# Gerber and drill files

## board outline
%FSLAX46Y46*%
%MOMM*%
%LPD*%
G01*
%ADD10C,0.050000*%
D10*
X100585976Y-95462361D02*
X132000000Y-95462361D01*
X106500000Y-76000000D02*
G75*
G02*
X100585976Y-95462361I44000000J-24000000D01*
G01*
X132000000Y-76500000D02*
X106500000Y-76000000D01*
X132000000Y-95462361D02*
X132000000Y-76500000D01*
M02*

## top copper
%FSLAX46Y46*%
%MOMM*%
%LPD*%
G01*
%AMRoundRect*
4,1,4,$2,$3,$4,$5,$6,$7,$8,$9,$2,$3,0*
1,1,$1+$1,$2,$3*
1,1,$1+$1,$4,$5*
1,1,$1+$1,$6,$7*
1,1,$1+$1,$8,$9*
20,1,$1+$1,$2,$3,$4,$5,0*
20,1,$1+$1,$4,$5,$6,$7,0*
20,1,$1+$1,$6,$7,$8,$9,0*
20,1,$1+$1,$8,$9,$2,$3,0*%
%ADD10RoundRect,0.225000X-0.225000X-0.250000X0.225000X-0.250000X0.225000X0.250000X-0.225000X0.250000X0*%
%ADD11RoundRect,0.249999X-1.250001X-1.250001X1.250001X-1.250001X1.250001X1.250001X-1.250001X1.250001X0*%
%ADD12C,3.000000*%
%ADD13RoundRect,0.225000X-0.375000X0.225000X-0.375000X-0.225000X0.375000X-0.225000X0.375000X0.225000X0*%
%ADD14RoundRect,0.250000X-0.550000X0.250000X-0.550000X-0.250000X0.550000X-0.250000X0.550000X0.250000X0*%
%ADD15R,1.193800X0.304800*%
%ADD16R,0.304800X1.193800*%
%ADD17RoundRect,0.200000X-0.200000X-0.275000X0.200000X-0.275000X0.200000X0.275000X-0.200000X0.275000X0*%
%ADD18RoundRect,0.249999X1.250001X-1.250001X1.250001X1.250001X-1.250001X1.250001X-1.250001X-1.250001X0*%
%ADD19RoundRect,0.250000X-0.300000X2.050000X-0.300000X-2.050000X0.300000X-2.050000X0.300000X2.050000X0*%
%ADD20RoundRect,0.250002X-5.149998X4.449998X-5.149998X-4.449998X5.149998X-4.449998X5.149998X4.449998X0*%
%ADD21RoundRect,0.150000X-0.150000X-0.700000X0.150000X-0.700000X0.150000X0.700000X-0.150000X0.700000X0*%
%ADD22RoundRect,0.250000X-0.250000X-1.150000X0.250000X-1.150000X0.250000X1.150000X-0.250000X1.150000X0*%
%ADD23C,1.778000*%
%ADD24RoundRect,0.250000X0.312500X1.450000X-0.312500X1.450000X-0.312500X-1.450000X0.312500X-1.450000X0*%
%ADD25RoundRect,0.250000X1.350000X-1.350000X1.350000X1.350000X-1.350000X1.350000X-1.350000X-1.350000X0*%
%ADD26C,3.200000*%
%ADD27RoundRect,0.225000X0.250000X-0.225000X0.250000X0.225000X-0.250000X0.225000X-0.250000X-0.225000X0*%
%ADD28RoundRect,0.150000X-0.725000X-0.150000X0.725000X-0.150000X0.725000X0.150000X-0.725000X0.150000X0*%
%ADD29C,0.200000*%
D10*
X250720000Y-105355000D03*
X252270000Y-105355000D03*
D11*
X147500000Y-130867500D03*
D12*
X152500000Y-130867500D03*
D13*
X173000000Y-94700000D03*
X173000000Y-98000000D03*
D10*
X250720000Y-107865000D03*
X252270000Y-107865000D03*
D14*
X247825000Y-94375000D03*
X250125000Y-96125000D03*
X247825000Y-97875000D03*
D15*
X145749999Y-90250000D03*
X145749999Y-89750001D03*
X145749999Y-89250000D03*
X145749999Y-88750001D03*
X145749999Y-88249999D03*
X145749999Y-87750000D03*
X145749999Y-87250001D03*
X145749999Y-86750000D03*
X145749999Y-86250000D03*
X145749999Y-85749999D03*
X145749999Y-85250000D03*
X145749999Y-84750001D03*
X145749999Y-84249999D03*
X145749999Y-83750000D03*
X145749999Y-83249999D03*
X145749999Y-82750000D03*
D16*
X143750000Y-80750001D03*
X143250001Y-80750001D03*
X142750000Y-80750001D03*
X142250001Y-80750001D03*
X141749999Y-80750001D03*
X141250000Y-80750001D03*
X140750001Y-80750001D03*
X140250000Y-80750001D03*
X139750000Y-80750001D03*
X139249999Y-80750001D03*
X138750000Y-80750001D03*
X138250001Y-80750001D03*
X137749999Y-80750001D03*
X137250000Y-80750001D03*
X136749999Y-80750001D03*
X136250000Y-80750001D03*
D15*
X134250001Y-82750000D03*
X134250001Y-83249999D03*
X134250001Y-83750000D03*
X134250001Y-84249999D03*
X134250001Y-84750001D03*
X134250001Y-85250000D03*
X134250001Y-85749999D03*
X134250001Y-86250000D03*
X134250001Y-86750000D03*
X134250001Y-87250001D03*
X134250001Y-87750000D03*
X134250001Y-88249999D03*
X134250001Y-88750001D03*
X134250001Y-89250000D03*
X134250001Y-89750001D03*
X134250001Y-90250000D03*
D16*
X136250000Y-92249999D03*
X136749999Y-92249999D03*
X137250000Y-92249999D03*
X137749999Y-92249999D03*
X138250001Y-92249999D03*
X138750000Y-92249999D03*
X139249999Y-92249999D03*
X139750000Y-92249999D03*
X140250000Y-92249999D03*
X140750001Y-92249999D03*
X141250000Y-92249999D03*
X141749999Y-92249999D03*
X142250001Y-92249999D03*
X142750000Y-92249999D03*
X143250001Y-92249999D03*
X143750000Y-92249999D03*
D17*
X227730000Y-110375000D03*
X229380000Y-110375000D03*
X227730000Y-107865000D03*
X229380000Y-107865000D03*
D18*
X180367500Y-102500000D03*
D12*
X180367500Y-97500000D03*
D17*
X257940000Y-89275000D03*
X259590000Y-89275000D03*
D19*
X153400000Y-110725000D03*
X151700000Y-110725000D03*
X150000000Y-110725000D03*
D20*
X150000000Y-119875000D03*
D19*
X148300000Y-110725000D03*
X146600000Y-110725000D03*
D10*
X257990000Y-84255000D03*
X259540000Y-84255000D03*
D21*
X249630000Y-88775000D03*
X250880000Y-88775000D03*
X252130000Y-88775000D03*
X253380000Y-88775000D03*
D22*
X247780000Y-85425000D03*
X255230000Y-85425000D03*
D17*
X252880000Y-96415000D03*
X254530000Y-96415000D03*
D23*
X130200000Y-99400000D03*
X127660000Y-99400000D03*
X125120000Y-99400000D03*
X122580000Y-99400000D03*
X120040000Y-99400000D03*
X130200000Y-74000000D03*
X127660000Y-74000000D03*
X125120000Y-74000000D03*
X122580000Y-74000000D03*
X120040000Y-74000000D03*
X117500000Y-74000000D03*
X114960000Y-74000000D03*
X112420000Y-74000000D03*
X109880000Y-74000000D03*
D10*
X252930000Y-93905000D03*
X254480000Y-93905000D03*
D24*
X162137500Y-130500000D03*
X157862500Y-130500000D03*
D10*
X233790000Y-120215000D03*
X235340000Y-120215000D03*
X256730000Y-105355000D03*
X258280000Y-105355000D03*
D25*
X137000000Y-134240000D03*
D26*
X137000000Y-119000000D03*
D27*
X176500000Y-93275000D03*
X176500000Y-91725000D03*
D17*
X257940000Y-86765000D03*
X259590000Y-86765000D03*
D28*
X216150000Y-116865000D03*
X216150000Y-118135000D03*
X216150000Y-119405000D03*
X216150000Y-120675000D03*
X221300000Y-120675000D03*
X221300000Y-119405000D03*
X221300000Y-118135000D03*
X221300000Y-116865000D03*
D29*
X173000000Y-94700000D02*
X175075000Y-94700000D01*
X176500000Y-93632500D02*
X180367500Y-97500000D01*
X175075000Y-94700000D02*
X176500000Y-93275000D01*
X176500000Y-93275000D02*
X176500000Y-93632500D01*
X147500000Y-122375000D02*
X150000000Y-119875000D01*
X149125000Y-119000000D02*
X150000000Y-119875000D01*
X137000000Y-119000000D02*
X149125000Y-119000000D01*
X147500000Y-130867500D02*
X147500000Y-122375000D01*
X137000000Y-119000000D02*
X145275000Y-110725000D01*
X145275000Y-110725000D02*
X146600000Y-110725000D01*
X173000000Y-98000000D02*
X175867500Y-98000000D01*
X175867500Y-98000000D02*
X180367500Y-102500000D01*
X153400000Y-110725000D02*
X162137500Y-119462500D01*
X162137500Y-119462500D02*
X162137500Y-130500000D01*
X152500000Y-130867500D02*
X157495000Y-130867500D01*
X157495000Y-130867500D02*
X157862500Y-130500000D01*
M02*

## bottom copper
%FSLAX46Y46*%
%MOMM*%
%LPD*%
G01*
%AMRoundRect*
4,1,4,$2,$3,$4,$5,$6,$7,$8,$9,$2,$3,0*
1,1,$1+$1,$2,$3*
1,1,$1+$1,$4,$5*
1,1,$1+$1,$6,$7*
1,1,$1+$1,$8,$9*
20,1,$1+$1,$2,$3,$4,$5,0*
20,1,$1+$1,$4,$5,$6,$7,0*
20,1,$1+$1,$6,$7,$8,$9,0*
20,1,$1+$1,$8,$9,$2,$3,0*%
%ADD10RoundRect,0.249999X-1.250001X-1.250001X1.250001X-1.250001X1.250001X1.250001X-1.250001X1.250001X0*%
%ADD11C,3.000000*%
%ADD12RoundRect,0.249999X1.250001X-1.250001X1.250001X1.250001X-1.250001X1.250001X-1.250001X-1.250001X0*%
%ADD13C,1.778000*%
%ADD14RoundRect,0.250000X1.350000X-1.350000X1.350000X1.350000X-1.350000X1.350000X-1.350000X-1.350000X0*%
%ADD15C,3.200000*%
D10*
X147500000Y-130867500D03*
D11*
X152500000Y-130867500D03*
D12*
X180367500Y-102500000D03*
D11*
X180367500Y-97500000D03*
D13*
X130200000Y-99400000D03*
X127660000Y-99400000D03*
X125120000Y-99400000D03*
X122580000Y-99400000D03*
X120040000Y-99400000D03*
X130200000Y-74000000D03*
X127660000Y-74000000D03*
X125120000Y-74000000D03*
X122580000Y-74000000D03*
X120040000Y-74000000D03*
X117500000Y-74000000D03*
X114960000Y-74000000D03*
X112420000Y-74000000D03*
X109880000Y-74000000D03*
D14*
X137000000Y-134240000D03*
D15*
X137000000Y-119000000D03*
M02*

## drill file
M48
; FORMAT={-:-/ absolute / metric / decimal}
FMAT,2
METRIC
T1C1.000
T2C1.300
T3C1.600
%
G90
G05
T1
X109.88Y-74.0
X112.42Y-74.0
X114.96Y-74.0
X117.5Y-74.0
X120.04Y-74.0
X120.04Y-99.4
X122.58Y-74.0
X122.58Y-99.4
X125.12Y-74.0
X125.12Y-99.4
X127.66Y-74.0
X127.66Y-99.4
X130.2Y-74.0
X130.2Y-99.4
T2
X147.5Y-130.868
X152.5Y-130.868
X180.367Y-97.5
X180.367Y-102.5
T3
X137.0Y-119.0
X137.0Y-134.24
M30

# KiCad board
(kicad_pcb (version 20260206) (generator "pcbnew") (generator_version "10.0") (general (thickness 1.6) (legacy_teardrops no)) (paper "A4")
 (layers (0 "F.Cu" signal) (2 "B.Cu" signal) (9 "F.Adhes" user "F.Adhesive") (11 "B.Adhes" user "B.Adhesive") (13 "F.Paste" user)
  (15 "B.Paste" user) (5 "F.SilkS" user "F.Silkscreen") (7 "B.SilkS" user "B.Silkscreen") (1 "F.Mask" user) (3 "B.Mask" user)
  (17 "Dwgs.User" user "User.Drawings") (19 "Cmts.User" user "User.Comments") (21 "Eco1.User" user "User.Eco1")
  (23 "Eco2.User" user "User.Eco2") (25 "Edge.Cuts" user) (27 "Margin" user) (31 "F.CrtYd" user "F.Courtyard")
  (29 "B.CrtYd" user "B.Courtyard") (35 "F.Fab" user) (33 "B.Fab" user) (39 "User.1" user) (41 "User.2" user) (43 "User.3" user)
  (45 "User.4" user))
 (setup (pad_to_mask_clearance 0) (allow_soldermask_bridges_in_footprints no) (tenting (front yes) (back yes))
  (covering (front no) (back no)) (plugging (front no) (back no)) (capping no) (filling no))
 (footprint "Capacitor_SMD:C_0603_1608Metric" (layer "F.Cu") (at 251.495 105.355)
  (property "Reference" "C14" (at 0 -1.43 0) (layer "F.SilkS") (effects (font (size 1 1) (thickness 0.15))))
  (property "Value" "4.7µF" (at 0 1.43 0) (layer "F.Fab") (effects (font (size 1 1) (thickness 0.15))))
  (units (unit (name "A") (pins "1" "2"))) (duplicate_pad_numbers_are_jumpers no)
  (pad "1" smd roundrect (at -0.775 0) (size 0.9 0.95) (layers "F.Cu" "F.Mask" "F.Paste") (roundrect_rratio 0.25) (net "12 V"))
  (pad "2" smd roundrect (at 0.775 0) (size 0.9 0.95) (layers "F.Cu" "F.Mask" "F.Paste") (roundrect_rratio 0.25) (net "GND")))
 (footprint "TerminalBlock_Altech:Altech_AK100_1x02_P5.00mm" (layer "F.Cu") (at 147.5 130.8675)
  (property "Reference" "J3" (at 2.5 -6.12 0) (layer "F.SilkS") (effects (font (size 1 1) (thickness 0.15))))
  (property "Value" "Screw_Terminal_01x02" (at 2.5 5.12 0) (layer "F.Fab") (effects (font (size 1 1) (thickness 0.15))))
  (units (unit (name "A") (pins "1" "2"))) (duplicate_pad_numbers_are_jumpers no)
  (pad "1" thru_hole roundrect (at 0 0) (size 3 3) (drill 1.3) (layers "*.Cu" "*.Mask") (remove_unused_layers no)
   (roundrect_rratio 0.083333) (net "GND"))
  (pad "2" thru_hole circle (at 5 0) (size 3 3) (drill 1.3) (layers "*.Cu" "*.Mask") (remove_unused_layers no) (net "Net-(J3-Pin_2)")))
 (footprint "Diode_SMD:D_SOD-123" (layer "F.Cu") (at 173 96.35 -90)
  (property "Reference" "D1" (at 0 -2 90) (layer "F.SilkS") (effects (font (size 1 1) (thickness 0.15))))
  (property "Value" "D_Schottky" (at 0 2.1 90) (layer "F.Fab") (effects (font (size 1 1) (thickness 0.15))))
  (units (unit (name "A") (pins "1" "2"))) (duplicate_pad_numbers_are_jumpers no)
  (pad "1" smd roundrect (at -1.65 0 270) (size 0.9 1.2) (layers "F.Cu" "F.Mask" "F.Paste") (roundrect_rratio 0.25) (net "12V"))
  (pad "2" smd roundrect (at 1.65 0 270) (size 0.9 1.2) (layers "F.Cu" "F.Mask" "F.Paste") (roundrect_rratio 0.25) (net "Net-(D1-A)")))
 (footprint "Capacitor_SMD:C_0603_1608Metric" (layer "F.Cu") (at 251.495 107.865)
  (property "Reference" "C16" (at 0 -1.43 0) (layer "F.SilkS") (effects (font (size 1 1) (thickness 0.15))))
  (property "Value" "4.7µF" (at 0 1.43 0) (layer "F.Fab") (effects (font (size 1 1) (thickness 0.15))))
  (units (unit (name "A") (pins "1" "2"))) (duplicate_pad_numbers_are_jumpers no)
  (pad "1" smd roundrect (at -0.775 0) (size 0.9 0.95) (layers "F.Cu" "F.Mask" "F.Paste") (roundrect_rratio 0.25) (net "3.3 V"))
  (pad "2" smd roundrect (at 0.775 0) (size 0.9 0.95) (layers "F.Cu" "F.Mask" "F.Paste") (roundrect_rratio 0.25) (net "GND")))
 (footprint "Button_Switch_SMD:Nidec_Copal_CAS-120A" (layer "F.Cu") (at 248.975 96.125)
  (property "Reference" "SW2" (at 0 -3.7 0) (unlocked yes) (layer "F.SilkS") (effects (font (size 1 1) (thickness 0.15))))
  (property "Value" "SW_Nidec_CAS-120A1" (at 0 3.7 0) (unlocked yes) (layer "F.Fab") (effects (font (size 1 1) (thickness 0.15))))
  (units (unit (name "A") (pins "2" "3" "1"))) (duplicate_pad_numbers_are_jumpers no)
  (pad "1" smd roundrect (at -1.15 -1.75 270) (size 1 1.6) (layers "F.Cu" "F.Mask" "F.Paste") (roundrect_rratio 0.25) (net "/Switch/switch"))
  (pad "2" smd roundrect (at 1.15 0 270) (size 1 1.6) (layers "F.Cu" "F.Mask" "F.Paste") (roundrect_rratio 0.25) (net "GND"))
  (pad "3" smd roundrect (at -1.15 1.75 270) (size 1 1.6) (layers "F.Cu" "F.Mask" "F.Paste") (roundrect_rratio 0.25)
   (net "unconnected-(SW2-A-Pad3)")))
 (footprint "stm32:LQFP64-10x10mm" (layer "F.Cu") (at 140 86.5 180)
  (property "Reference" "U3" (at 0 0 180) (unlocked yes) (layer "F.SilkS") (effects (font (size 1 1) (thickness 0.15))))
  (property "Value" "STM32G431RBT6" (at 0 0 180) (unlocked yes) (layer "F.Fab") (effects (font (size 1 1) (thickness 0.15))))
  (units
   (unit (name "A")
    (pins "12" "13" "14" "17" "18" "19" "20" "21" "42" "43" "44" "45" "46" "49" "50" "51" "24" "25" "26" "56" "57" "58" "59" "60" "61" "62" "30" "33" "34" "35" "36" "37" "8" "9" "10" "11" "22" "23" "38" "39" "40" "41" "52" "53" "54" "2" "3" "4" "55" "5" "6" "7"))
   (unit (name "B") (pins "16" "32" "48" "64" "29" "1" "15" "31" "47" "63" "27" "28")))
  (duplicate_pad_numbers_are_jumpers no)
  (pad "1" smd rect (at -5.749999 -3.75 180) (size 1.1938 0.3048) (layers "F.Cu" "F.Mask" "F.Paste") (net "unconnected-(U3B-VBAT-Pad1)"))
  (pad "2" smd rect (at -5.749999 -3.250001 180) (size 1.1938 0.3048) (layers "F.Cu" "F.Mask" "F.Paste") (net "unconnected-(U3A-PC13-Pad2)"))
  (pad "3" smd rect (at -5.749999 -2.75 180) (size 1.1938 0.3048) (layers "F.Cu" "F.Mask" "F.Paste")
   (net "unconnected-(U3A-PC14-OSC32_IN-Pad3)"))
  (pad "4" smd rect (at -5.749999 -2.250001 180) (size 1.1938 0.3048) (layers "F.Cu" "F.Mask" "F.Paste")
   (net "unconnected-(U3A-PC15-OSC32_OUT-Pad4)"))
  (pad "5" smd rect (at -5.749999 -1.749999 180) (size 1.1938 0.3048) (layers "F.Cu" "F.Mask" "F.Paste")
   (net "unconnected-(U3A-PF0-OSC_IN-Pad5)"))
  (pad "6" smd rect (at -5.749999 -1.25 180) (size 1.1938 0.3048) (layers "F.Cu" "F.Mask" "F.Paste")
   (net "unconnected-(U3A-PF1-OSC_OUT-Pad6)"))
  (pad "7" smd rect (at -5.749999 -0.750001 180) (size 1.1938 0.3048) (layers "F.Cu" "F.Mask" "F.Paste")
   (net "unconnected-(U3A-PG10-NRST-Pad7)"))
  (pad "8" smd rect (at -5.749999 -0.25 180) (size 1.1938 0.3048) (layers "F.Cu" "F.Mask" "F.Paste") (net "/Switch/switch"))
  (pad "9" smd rect (at -5.749999 0.25 180) (size 1.1938 0.3048) (layers "F.Cu" "F.Mask" "F.Paste") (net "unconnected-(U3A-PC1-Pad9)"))
  (pad "10" smd rect (at -5.749999 0.750001 180) (size 1.1938 0.3048) (layers "F.Cu" "F.Mask" "F.Paste") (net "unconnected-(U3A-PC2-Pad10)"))
  (pad "11" smd rect (at -5.749999 1.25 180) (size 1.1938 0.3048) (layers "F.Cu" "F.Mask" "F.Paste") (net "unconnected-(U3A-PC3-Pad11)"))
  (pad "12" smd rect (at -5.749999 1.749999 180) (size 1.1938 0.3048) (layers "F.Cu" "F.Mask" "F.Paste") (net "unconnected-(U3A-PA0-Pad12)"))
  (pad "13" smd rect (at -5.749999 2.250001 180) (size 1.1938 0.3048) (layers "F.Cu" "F.Mask" "F.Paste") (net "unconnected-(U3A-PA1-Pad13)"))
  (pad "14" smd rect (at -5.749999 2.75 180) (size 1.1938 0.3048) (layers "F.Cu" "F.Mask" "F.Paste") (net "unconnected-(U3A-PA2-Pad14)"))
  (pad "15" smd rect (at -5.749999 3.250001 180) (size 1.1938 0.3048) (layers "F.Cu" "F.Mask" "F.Paste") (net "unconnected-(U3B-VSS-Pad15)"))
  (pad "16" smd rect (at -5.749999 3.75 180) (size 1.1938 0.3048) (layers "F.Cu" "F.Mask" "F.Paste") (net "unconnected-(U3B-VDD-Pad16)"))
  (pad "17" smd rect (at -3.75 5.749999 270) (size 1.1938 0.3048) (layers "F.Cu" "F.Mask" "F.Paste") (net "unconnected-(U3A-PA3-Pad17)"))
  (pad "18" smd rect (at -3.250001 5.749999 270) (size 1.1938 0.3048) (layers "F.Cu" "F.Mask" "F.Paste") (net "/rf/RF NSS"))
  (pad "19" smd rect (at -2.75 5.749999 270) (size 1.1938 0.3048) (layers "F.Cu" "F.Mask" "F.Paste") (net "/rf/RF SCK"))
  (pad "20" smd rect (at -2.250001 5.749999 270) (size 1.1938 0.3048) (layers "F.Cu" "F.Mask" "F.Paste") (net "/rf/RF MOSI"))
  (pad "21" smd rect (at -1.749999 5.749999 270) (size 1.1938 0.3048) (layers "F.Cu" "F.Mask" "F.Paste") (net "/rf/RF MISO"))
  (pad "22" smd rect (at -1.25 5.749999 270) (size 1.1938 0.3048) (layers "F.Cu" "F.Mask" "F.Paste") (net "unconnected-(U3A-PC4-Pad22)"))
  (pad "23" smd rect (at -0.750001 5.749999 270) (size 1.1938 0.3048) (layers "F.Cu" "F.Mask" "F.Paste") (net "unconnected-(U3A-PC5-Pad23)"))
  (pad "24" smd rect (at -0.25 5.749999 270) (size 1.1938 0.3048) (layers "F.Cu" "F.Mask" "F.Paste") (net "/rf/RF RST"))
  (pad "25" smd rect (at 0.25 5.749999 270) (size 1.1938 0.3048) (layers "F.Cu" "F.Mask" "F.Paste") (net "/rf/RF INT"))
  (pad "26" smd rect (at 0.750001 5.749999 270) (size 1.1938 0.3048) (layers "F.Cu" "F.Mask" "F.Paste") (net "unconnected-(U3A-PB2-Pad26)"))
  (pad "27" smd rect (at 1.25 5.749999 270) (size 1.1938 0.3048) (layers "F.Cu" "F.Mask" "F.Paste") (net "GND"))
  (pad "28" smd rect (at 1.749999 5.749999 270) (size 1.1938 0.3048) (layers "F.Cu" "F.Mask" "F.Paste") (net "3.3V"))
  (pad "29" smd rect (at 2.250001 5.749999 270) (size 1.1938 0.3048) (layers "F.Cu" "F.Mask" "F.Paste") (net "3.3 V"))
  (pad "30" smd rect (at 2.75 5.749999 270) (size 1.1938 0.3048) (layers "F.Cu" "F.Mask" "F.Paste") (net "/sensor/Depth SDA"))
  (pad "31" smd rect (at 3.250001 5.749999 270) (size 1.1938 0.3048) (layers "F.Cu" "F.Mask" "F.Paste") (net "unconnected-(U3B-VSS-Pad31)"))
  (pad "32" smd rect (at 3.75 5.749999 270) (size 1.1938 0.3048) (layers "F.Cu" "F.Mask" "F.Paste") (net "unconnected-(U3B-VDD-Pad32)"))
  (pad "33" smd rect (at 5.749999 3.75 180) (size 1.1938 0.3048) (layers "F.Cu" "F.Mask" "F.Paste") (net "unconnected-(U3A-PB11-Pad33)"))
  (pad "34" smd rect (at 5.749999 3.250001 180) (size 1.1938 0.3048) (layers "F.Cu" "F.Mask" "F.Paste") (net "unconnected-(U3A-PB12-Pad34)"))
  (pad "35" smd rect (at 5.749999 2.75 180) (size 1.1938 0.3048) (layers "F.Cu" "F.Mask" "F.Paste") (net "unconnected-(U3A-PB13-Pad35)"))
  (pad "36" smd rect (at 5.749999 2.250001 180) (size 1.1938 0.3048) (layers "F.Cu" "F.Mask" "F.Paste") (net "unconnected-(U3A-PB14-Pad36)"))
  (pad "37" smd rect (at 5.749999 1.749999 180) (size 1.1938 0.3048) (layers "F.Cu" "F.Mask" "F.Paste") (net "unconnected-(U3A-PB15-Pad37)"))
  (pad "38" smd rect (at 5.749999 1.25 180) (size 1.1938 0.3048) (layers "F.Cu" "F.Mask" "F.Paste") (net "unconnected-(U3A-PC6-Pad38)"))
  (pad "39" smd rect (at 5.749999 0.750001 180) (size 1.1938 0.3048) (layers "F.Cu" "F.Mask" "F.Paste") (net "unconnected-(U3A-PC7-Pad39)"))
  (pad "40" smd rect (at 5.749999 0.25 180) (size 1.1938 0.3048) (layers "F.Cu" "F.Mask" "F.Paste") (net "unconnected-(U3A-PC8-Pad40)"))
  (pad "41" smd rect (at 5.749999 -0.25 180) (size 1.1938 0.3048) (layers "F.Cu" "F.Mask" "F.Paste") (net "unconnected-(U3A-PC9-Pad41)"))
  (pad "42" smd rect (at 5.749999 -0.750001 180) (size 1.1938 0.3048) (layers "F.Cu" "F.Mask" "F.Paste") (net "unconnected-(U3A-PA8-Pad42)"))
  (pad "43" smd rect (at 5.749999 -1.25 180) (size 1.1938 0.3048) (layers "F.Cu" "F.Mask" "F.Paste") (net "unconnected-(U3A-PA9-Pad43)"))
  (pad "44" smd rect (at 5.749999 -1.749999 180) (size 1.1938 0.3048) (layers "F.Cu" "F.Mask" "F.Paste") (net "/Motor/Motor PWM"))
  (pad "45" smd rect (at 5.749999 -2.250001 180) (size 1.1938 0.3048) (layers "F.Cu" "F.Mask" "F.Paste")
   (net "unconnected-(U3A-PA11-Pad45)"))
  (pad "46" smd rect (at 5.749999 -2.75 180) (size 1.1938 0.3048) (layers "F.Cu" "F.Mask" "F.Paste") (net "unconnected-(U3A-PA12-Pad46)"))
  (pad "47" smd rect (at 5.749999 -3.250001 180) (size 1.1938 0.3048) (layers "F.Cu" "F.Mask" "F.Paste") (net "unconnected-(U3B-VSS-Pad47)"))
  (pad "48" smd rect (at 5.749999 -3.75 180) (size 1.1938 0.3048) (layers "F.Cu" "F.Mask" "F.Paste") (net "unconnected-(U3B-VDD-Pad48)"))
  (pad "49" smd rect (at 3.75 -5.749999 270) (size 1.1938 0.3048) (layers "F.Cu" "F.Mask" "F.Paste") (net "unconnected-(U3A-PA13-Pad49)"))
  (pad "50" smd rect (at 3.250001 -5.749999 270) (size 1.1938 0.3048) (layers "F.Cu" "F.Mask" "F.Paste")
   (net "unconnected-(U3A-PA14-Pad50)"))
  (pad "51" smd rect (at 2.75 -5.749999 270) (size 1.1938 0.3048) (layers "F.Cu" "F.Mask" "F.Paste") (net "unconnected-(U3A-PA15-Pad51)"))
  (pad "52" smd rect (at 2.250001 -5.749999 270) (size 1.1938 0.3048) (layers "F.Cu" "F.Mask" "F.Paste")
   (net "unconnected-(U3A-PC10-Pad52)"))
  (pad "53" smd rect (at 1.749999 -5.749999 270) (size 1.1938 0.3048) (layers "F.Cu" "F.Mask" "F.Paste")
   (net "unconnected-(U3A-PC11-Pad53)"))
  (pad "54" smd rect (at 1.25 -5.749999 270) (size 1.1938 0.3048) (layers "F.Cu" "F.Mask" "F.Paste") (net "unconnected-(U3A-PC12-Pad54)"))
  (pad "55" smd rect (at 0.750001 -5.749999 270) (size 1.1938 0.3048) (layers "F.Cu" "F.Mask" "F.Paste") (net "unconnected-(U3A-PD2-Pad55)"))
  (pad "56" smd rect (at 0.25 -5.749999 270) (size 1.1938 0.3048) (layers "F.Cu" "F.Mask" "F.Paste") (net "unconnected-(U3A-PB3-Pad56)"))
  (pad "57" smd rect (at -0.25 -5.749999 270) (size 1.1938 0.3048) (layers "F.Cu" "F.Mask" "F.Paste") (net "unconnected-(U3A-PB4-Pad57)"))
  (pad "58" smd rect (at -0.750001 -5.749999 270) (size 1.1938 0.3048) (layers "F.Cu" "F.Mask" "F.Paste")
   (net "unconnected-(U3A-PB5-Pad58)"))
  (pad "59" smd rect (at -1.25 -5.749999 270) (size 1.1938 0.3048) (layers "F.Cu" "F.Mask" "F.Paste") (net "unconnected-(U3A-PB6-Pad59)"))
  (pad "60" smd rect (at -1.749999 -5.749999 270) (size 1.1938 0.3048) (layers "F.Cu" "F.Mask" "F.Paste")
   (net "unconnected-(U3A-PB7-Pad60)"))
  (pad "61" smd rect (at -2.250001 -5.749999 270) (size 1.1938 0.3048) (layers "F.Cu" "F.Mask" "F.Paste")
   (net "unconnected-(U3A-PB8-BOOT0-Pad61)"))
  (pad "62" smd rect (at -2.75 -5.749999 270) (size 1.1938 0.3048) (layers "F.Cu" "F.Mask" "F.Paste") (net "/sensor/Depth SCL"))
  (pad "63" smd rect (at -3.250001 -5.749999 270) (size 1.1938 0.3048) (layers "F.Cu" "F.Mask" "F.Paste") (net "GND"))
  (pad "64" smd rect (at -3.75 -5.749999 270) (size 1.1938 0.3048) (layers "F.Cu" "F.Mask" "F.Paste") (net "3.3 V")))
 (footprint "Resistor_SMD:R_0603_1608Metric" (layer "F.Cu") (at 228.555 110.375)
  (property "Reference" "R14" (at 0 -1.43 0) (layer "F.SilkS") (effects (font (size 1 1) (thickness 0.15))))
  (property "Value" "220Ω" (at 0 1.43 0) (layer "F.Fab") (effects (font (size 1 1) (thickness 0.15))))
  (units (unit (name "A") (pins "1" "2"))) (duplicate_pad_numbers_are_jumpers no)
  (pad "1" smd roundrect (at -0.825 0) (size 0.8 0.95) (layers "F.Cu" "F.Mask" "F.Paste") (roundrect_rratio 0.25) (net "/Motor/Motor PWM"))
  (pad "2" smd roundrect (at 0.825 0) (size 0.8 0.95) (layers "F.Cu" "F.Mask" "F.Paste") (roundrect_rratio 0.25) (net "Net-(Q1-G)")))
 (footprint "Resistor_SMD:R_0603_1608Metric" (layer "F.Cu") (at 228.555 107.865)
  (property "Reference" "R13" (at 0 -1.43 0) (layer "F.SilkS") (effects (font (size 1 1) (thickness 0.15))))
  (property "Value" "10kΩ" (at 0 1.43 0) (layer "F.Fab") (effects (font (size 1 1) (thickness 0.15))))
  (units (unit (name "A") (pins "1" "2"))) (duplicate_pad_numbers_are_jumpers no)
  (pad "1" smd roundrect (at -0.825 0) (size 0.8 0.95) (layers "F.Cu" "F.Mask" "F.Paste") (roundrect_rratio 0.25) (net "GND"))
  (pad "2" smd roundrect (at 0.825 0) (size 0.8 0.95) (layers "F.Cu" "F.Mask" "F.Paste") (roundrect_rratio 0.25) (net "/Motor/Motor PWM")))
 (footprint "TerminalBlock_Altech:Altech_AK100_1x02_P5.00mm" (layer "F.Cu") (at 180.3675 102.5 90)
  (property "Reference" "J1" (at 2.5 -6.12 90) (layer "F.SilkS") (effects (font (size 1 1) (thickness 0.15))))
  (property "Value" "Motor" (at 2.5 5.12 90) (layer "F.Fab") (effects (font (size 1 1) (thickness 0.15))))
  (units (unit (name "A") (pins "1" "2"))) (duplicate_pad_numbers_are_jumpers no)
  (pad "1" thru_hole roundrect (at 0 0 90) (size 3 3) (drill 1.3) (layers "*.Cu" "*.Mask") (remove_unused_layers no)
   (roundrect_rratio 0.083333) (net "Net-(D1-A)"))
  (pad "2" thru_hole circle (at 5 0 90) (size 3 3) (drill 1.3) (layers "*.Cu" "*.Mask") (remove_unused_layers no) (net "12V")))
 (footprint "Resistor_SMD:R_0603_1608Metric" (layer "F.Cu") (at 258.765 89.275)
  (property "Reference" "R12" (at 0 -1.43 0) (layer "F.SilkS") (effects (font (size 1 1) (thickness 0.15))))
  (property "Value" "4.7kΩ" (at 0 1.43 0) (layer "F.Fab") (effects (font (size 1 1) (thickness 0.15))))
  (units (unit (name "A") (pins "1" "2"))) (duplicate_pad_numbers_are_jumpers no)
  (pad "1" smd roundrect (at -0.825 0) (size 0.8 0.95) (layers "F.Cu" "F.Mask" "F.Paste") (roundrect_rratio 0.25) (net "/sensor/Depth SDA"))
  (pad "2" smd roundrect (at 0.825 0) (size 0.8 0.95) (layers "F.Cu" "F.Mask" "F.Paste") (roundrect_rratio 0.25) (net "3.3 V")))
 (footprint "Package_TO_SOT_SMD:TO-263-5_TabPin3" (layer "F.Cu") (at 150 118.375 -90)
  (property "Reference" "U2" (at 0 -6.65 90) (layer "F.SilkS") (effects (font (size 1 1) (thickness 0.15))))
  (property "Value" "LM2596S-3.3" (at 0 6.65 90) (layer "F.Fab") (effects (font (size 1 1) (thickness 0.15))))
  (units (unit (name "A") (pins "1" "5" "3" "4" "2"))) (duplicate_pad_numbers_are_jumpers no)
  (pad "" smd roundrect (at -0.925 -2.775 270) (size 4.55 5.25) (layers "F.Paste") (roundrect_rratio 0.054945))
  (pad "" smd roundrect (at -0.925 2.775 270) (size 4.55 5.25) (layers "F.Paste") (roundrect_rratio 0.054945))
  (pad "" smd roundrect (at 3.925 -2.775 270) (size 4.55 5.25) (layers "F.Paste") (roundrect_rratio 0.054945))
  (pad "" smd roundrect (at 3.925 2.775 270) (size 4.55 5.25) (layers "F.Paste") (roundrect_rratio 0.054945))
  (pad "1" smd roundrect (at -7.65 -3.4 270) (size 4.6 1.1) (layers "F.Cu" "F.Mask" "F.Paste") (roundrect_rratio 0.227273) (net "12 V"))
  (pad "2" smd roundrect (at -7.65 -1.7 270) (size 4.6 1.1) (layers "F.Cu" "F.Mask" "F.Paste") (roundrect_rratio 0.227273)
   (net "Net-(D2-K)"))
  (pad "3" smd roundrect (at -7.65 0 270) (size 4.6 1.1) (layers "F.Cu" "F.Mask" "F.Paste") (roundrect_rratio 0.227273) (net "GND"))
  (pad "3" smd roundrect (at 1.5 0 270) (size 9.4 10.8) (layers "F.Cu" "F.Mask") (roundrect_rratio 0.026596) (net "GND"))
  (pad "4" smd roundrect (at -7.65 1.7 270) (size 4.6 1.1) (layers "F.Cu" "F.Mask" "F.Paste") (roundrect_rratio 0.227273) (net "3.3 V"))
  (pad "5" smd roundrect (at -7.65 3.4 270) (size 4.6 1.1) (layers "F.Cu" "F.Mask" "F.Paste") (roundrect_rratio 0.227273) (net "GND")))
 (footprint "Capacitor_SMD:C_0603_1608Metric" (layer "F.Cu") (at 258.765 84.255)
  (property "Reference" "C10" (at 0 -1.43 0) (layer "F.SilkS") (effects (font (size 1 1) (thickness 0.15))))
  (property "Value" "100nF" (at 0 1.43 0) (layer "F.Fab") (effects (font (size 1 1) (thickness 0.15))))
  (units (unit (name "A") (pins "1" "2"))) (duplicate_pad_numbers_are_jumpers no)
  (pad "1" smd roundrect (at -0.775 0) (size 0.9 0.95) (layers "F.Cu" "F.Mask" "F.Paste") (roundrect_rratio 0.25) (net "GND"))
  (pad "2" smd roundrect (at 0.775 0) (size 0.9 0.95) (layers "F.Cu" "F.Mask" "F.Paste") (roundrect_rratio 0.25) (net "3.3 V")))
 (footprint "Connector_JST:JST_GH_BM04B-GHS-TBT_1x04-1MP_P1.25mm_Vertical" (layer "F.Cu") (at 251.505 86.825)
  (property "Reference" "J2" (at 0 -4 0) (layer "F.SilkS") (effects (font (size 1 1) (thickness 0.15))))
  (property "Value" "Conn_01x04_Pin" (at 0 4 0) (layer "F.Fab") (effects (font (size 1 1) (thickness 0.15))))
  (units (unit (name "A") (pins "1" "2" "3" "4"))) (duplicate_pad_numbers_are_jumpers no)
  (pad "1" smd roundrect (at -1.875 1.95) (size 0.6 1.7) (layers "F.Cu" "F.Mask" "F.Paste") (roundrect_rratio 0.25) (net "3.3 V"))
  (pad "2" smd roundrect (at -0.625 1.95) (size 0.6 1.7) (layers "F.Cu" "F.Mask" "F.Paste") (roundrect_rratio 0.25)
   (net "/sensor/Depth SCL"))
  (pad "3" smd roundrect (at 0.625 1.95) (size 0.6 1.7) (layers "F.Cu" "F.Mask" "F.Paste") (roundrect_rratio 0.25) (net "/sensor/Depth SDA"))
  (pad "4" smd roundrect (at 1.875 1.95) (size 0.6 1.7) (layers "F.Cu" "F.Mask" "F.Paste") (roundrect_rratio 0.25) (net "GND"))
  (pad "MP" smd roundrect (at -3.725 -1.4) (size 1 2.8) (layers "F.Cu" "F.Mask" "F.Paste") (roundrect_rratio 0.25))
  (pad "MP" smd roundrect (at 3.725 -1.4) (size 1 2.8) (layers "F.Cu" "F.Mask" "F.Paste") (roundrect_rratio 0.25)))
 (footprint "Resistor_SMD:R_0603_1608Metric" (layer "F.Cu") (at 253.705 96.415)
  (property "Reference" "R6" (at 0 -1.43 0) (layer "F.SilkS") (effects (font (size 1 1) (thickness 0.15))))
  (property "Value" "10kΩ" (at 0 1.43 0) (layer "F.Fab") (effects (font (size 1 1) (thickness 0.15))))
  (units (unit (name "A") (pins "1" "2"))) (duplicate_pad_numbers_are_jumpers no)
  (pad "1" smd roundrect (at -0.825 0) (size 0.8 0.95) (layers "F.Cu" "F.Mask" "F.Paste") (roundrect_rratio 0.25) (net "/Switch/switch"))
  (pad "2" smd roundrect (at 0.825 0) (size 0.8 0.95) (layers "F.Cu" "F.Mask" "F.Paste") (roundrect_rratio 0.25) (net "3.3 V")))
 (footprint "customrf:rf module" (layer "F.Cu") (at 130.2 99.4 180)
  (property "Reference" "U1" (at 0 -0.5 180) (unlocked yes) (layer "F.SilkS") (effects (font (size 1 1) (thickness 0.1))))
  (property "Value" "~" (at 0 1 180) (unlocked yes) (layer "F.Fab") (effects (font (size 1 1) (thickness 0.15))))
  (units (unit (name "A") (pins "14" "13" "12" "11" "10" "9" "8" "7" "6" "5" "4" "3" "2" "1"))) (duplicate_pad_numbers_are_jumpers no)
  (pad "1" thru_hole circle (at 0 0 270) (size 1.778 1.778) (drill 1) (layers "*.Cu" "*.Mask") (remove_unused_layers no)
   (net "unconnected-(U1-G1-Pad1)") (solder_mask_margin 0.0508) (thermal_bridge_angle 0))
  (pad "2" thru_hole circle (at 2.54 0 270) (size 1.778 1.778) (drill 1) (layers "*.Cu" "*.Mask") (remove_unused_layers no)
   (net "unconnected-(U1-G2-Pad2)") (solder_mask_margin 0.0508) (thermal_bridge_angle 0))
  (pad "3" thru_hole circle (at 5.08 0 270) (size 1.778 1.778) (drill 1) (layers "*.Cu" "*.Mask") (remove_unused_layers no)
   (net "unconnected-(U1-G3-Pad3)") (solder_mask_margin 0.0508) (thermal_bridge_angle 0))
  (pad "4" thru_hole circle (at 7.62 0 270) (size 1.778 1.778) (drill 1) (layers "*.Cu" "*.Mask") (remove_unused_layers no)
   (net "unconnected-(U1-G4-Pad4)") (solder_mask_margin 0.0508) (thermal_bridge_angle 0))
  (pad "5" thru_hole circle (at 10.16 0 270) (size 1.778 1.778) (drill 1) (layers "*.Cu" "*.Mask") (remove_unused_layers no)
   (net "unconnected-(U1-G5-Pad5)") (solder_mask_margin 0.0508) (thermal_bridge_angle 0))
  (pad "6" thru_hole circle (at 0 25.4 270) (size 1.778 1.778) (drill 1) (layers "*.Cu" "*.Mask") (remove_unused_layers no) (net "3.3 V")
   (solder_mask_margin 0.0508) (thermal_bridge_angle 0))
  (pad "7" thru_hole circle (at 2.54 25.4 270) (size 1.778 1.778) (drill 1) (layers "*.Cu" "*.Mask") (remove_unused_layers no) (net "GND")
   (solder_mask_margin 0.0508) (thermal_bridge_angle 0))
  (pad "8" thru_hole circle (at 5.08 25.4 270) (size 1.778 1.778) (drill 1) (layers "*.Cu" "*.Mask") (remove_unused_layers no)
   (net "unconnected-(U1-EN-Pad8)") (solder_mask_margin 0.0508) (thermal_bridge_angle 0))
  (pad "9" thru_hole circle (at 7.62 25.4 270) (size 1.778 1.778) (drill 1) (layers "*.Cu" "*.Mask") (remove_unused_layers no)
   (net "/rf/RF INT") (solder_mask_margin 0.0508) (thermal_bridge_angle 0))
  (pad "10" thru_hole circle (at 10.16 25.4 270) (size 1.778 1.778) (drill 1) (layers "*.Cu" "*.Mask") (remove_unused_layers no)
   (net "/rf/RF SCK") (solder_mask_margin 0.0508) (thermal_bridge_angle 0))
  (pad "11" thru_hole circle (at 12.7 25.4 270) (size 1.778 1.778) (drill 1) (layers "*.Cu" "*.Mask") (remove_unused_layers no)
   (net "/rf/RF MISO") (solder_mask_margin 0.0508) (thermal_bridge_angle 0))
  (pad "12" thru_hole circle (at 15.24 25.4 270) (size 1.778 1.778) (drill 1) (layers "*.Cu" "*.Mask") (remove_unused_layers no)
   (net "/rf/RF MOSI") (solder_mask_margin 0.0508) (thermal_bridge_angle 0))
  (pad "13" thru_hole circle (at 17.78 25.4 270) (size 1.778 1.778) (drill 1) (layers "*.Cu" "*.Mask") (remove_unused_layers no)
   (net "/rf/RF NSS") (solder_mask_margin 0.0508) (thermal_bridge_angle 0))
  (pad "14" thru_hole circle (at 20.32 25.4 270) (size 1.778 1.778) (drill 1) (layers "*.Cu" "*.Mask") (remove_unused_layers no)
   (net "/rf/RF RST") (solder_mask_margin 0.0508) (thermal_bridge_angle 0)))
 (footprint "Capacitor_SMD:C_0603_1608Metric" (layer "F.Cu") (at 253.705 93.905)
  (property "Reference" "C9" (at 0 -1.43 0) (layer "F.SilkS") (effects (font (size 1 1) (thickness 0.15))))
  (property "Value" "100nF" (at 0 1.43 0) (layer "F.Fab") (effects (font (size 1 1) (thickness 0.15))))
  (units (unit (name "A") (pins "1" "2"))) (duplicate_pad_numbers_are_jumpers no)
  (pad "1" smd roundrect (at -0.775 0) (size 0.9 0.95) (layers "F.Cu" "F.Mask" "F.Paste") (roundrect_rratio 0.25) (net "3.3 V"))
  (pad "2" smd roundrect (at 0.775 0) (size 0.9 0.95) (layers "F.Cu" "F.Mask" "F.Paste") (roundrect_rratio 0.25) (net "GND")))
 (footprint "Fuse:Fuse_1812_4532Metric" (layer "F.Cu") (at 160 130.5 180)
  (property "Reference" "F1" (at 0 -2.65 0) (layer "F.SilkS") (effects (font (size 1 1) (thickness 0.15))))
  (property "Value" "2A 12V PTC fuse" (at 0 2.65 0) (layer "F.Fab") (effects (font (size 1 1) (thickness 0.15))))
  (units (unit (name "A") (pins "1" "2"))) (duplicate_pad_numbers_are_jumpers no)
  (pad "1" smd roundrect (at -2.1375 0 180) (size 1.125 3.4) (layers "F.Cu" "F.Mask" "F.Paste") (roundrect_rratio 0.222222) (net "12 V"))
  (pad "2" smd roundrect (at 2.1375 0 180) (size 1.125 3.4) (layers "F.Cu" "F.Mask" "F.Paste") (roundrect_rratio 0.222222)
   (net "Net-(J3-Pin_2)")))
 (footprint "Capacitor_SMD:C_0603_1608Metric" (layer "F.Cu") (at 234.565 120.215)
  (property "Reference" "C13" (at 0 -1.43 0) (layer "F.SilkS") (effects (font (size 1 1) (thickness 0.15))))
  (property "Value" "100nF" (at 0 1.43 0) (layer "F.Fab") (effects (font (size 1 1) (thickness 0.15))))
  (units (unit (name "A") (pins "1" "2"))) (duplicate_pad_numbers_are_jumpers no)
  (pad "1" smd roundrect (at -0.775 0) (size 0.9 0.95) (layers "F.Cu" "F.Mask" "F.Paste") (roundrect_rratio 0.25) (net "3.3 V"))
  (pad "2" smd roundrect (at 0.775 0) (size 0.9 0.95) (layers "F.Cu" "F.Mask" "F.Paste") (roundrect_rratio 0.25) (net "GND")))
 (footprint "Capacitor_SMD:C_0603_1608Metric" (layer "F.Cu") (at 257.505 105.355)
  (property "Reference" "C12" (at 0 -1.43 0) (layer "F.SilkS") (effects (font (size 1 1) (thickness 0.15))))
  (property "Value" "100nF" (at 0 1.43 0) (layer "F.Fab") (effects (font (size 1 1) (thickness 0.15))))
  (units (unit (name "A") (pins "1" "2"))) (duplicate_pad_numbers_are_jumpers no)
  (pad "1" smd roundrect (at -0.775 0) (size 0.9 0.95) (layers "F.Cu" "F.Mask" "F.Paste") (roundrect_rratio 0.25) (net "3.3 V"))
  (pad "2" smd roundrect (at 0.775 0) (size 0.9 0.95) (layers "F.Cu" "F.Mask" "F.Paste") (roundrect_rratio 0.25) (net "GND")))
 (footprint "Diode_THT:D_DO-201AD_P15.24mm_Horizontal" (layer "F.Cu") (at 137 134.24 90)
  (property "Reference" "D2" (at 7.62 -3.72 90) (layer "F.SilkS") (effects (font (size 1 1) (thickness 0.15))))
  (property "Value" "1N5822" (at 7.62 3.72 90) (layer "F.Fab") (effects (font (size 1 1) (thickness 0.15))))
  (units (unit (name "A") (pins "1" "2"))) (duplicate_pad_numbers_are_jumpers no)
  (pad "1" thru_hole roundrect (at 0 0 90) (size 3.2 3.2) (drill 1.6) (layers "*.Cu" "*.Mask") (remove_unused_layers no)
   (roundrect_rratio 0.078125) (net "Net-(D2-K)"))
  (pad "2" thru_hole circle (at 15.24 0 90) (size 3.2 3.2) (drill 1.6) (layers "*.Cu" "*.Mask") (remove_unused_layers no) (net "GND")))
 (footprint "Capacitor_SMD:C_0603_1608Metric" (layer "F.Cu") (at 176.5 92.5 90)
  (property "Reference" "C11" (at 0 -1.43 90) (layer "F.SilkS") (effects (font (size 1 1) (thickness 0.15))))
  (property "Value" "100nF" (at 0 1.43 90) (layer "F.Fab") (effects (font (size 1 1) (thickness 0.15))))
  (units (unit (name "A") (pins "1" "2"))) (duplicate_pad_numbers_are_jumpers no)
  (pad "1" smd roundrect (at -0.775 0 90) (size 0.9 0.95) (layers "F.Cu" "F.Mask" "F.Paste") (roundrect_rratio 0.25) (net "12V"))
  (pad "2" smd roundrect (at 0.775 0 90) (size 0.9 0.95) (layers "F.Cu" "F.Mask" "F.Paste") (roundrect_rratio 0.25) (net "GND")))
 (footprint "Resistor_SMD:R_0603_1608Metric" (layer "F.Cu") (at 258.765 86.765)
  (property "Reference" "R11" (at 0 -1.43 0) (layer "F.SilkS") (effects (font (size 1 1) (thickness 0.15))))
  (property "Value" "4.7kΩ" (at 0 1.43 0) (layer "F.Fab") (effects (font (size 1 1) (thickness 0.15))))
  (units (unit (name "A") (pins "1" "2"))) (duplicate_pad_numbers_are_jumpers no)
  (pad "1" smd roundrect (at -0.825 0) (size 0.8 0.95) (layers "F.Cu" "F.Mask" "F.Paste") (roundrect_rratio 0.25) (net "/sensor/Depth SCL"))
  (pad "2" smd roundrect (at 0.825 0) (size 0.8 0.95) (layers "F.Cu" "F.Mask" "F.Paste") (roundrect_rratio 0.25) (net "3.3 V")))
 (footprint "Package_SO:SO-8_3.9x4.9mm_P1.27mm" (layer "F.Cu") (at 218.725 118.77)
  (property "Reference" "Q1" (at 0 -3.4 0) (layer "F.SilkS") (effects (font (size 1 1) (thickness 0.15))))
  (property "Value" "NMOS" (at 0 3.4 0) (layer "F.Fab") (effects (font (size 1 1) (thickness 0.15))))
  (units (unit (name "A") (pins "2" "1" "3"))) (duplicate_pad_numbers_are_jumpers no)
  (pad "1" smd roundrect (at -2.575 -1.905) (size 1.75 0.6) (layers "F.Cu" "F.Mask" "F.Paste") (roundrect_rratio 0.25) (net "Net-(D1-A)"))
  (pad "2" smd roundrect (at -2.575 -0.635) (size 1.75 0.6) (layers "F.Cu" "F.Mask" "F.Paste") (roundrect_rratio 0.25) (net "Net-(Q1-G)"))
  (pad "3" smd roundrect (at -2.575 0.635) (size 1.75 0.6) (layers "F.Cu" "F.Mask" "F.Paste") (roundrect_rratio 0.25) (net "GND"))
  (pad "4" smd roundrect (at -2.575 1.905) (size 1.75 0.6) (layers "F.Cu" "F.Mask" "F.Paste") (roundrect_rratio 0.25))
  (pad "5" smd roundrect (at 2.575 1.905) (size 1.75 0.6) (layers "F.Cu" "F.Mask" "F.Paste") (roundrect_rratio 0.25))
  (pad "6" smd roundrect (at 2.575 0.635) (size 1.75 0.6) (layers "F.Cu" "F.Mask" "F.Paste") (roundrect_rratio 0.25))
  (pad "7" smd roundrect (at 2.575 -0.635) (size 1.75 0.6) (layers "F.Cu" "F.Mask" "F.Paste") (roundrect_rratio 0.25))
  (pad "8" smd roundrect (at 2.575 -1.905) (size 1.75 0.6) (layers "F.Cu" "F.Mask" "F.Paste") (roundrect_rratio 0.25)))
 (gr_line (start 100.585976 95.462361) (end 132 95.462361) (stroke (width 0.05) (type default)) (layer "Edge.Cuts"))
 (gr_arc (start 106.5 76) (mid 198.454738 114.571998) (end 100.585976 95.462361) (stroke (width 0.05) (type default)) (layer "Edge.Cuts"))
 (gr_line (start 132 76.5) (end 106.5 76) (stroke (width 0.05) (type default)) (layer "Edge.Cuts"))
 (gr_line (start 132 95.462361) (end 132 76.5) (stroke (width 0.05) (type default)) (layer "Edge.Cuts"))
 (segment (start 173 94.7) (end 175.075 94.7) (width 0.2) (layer "F.Cu") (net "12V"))
 (segment (start 176.5 93.6325) (end 180.3675 97.5) (width 0.2) (layer "F.Cu") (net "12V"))
 (segment (start 175.075 94.7) (end 176.5 93.275) (width 0.2) (layer "F.Cu") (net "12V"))
 (segment (start 176.5 93.275) (end 176.5 93.6325) (width 0.2) (layer "F.Cu") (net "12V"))
 (segment (start 147.5 122.375) (end 150 119.875) (width 0.2) (layer "F.Cu") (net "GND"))
 (segment (start 149.125 119) (end 150 119.875) (width 0.2) (layer "F.Cu") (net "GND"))
 (segment (start 137 119) (end 149.125 119) (width 0.2) (layer "F.Cu") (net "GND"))
 (segment (start 147.5 130.8675) (end 147.5 122.375) (width 0.2) (layer "F.Cu") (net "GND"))
 (segment (start 137 119) (end 145.275 110.725) (width 0.2) (layer "F.Cu") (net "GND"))
 (segment (start 145.275 110.725) (end 146.6 110.725) (width 0.2) (layer "F.Cu") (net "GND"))
 (segment (start 173 98) (end 175.8675 98) (width 0.2) (layer "F.Cu") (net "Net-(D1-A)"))
 (segment (start 175.8675 98) (end 180.3675 102.5) (width 0.2) (layer "F.Cu") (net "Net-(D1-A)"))
 (segment (start 153.4 110.725) (end 162.1375 119.4625) (width 0.2) (layer "F.Cu") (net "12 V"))
 (segment (start 162.1375 119.4625) (end 162.1375 130.5) (width 0.2) (layer "F.Cu") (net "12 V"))
 (segment (start 152.5 130.8675) (end 157.495 130.8675) (width 0.2) (layer "F.Cu") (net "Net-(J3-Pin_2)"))
 (segment (start 157.495 130.8675) (end 157.8625 130.5) (width 0.2) (layer "F.Cu") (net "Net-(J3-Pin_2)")))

